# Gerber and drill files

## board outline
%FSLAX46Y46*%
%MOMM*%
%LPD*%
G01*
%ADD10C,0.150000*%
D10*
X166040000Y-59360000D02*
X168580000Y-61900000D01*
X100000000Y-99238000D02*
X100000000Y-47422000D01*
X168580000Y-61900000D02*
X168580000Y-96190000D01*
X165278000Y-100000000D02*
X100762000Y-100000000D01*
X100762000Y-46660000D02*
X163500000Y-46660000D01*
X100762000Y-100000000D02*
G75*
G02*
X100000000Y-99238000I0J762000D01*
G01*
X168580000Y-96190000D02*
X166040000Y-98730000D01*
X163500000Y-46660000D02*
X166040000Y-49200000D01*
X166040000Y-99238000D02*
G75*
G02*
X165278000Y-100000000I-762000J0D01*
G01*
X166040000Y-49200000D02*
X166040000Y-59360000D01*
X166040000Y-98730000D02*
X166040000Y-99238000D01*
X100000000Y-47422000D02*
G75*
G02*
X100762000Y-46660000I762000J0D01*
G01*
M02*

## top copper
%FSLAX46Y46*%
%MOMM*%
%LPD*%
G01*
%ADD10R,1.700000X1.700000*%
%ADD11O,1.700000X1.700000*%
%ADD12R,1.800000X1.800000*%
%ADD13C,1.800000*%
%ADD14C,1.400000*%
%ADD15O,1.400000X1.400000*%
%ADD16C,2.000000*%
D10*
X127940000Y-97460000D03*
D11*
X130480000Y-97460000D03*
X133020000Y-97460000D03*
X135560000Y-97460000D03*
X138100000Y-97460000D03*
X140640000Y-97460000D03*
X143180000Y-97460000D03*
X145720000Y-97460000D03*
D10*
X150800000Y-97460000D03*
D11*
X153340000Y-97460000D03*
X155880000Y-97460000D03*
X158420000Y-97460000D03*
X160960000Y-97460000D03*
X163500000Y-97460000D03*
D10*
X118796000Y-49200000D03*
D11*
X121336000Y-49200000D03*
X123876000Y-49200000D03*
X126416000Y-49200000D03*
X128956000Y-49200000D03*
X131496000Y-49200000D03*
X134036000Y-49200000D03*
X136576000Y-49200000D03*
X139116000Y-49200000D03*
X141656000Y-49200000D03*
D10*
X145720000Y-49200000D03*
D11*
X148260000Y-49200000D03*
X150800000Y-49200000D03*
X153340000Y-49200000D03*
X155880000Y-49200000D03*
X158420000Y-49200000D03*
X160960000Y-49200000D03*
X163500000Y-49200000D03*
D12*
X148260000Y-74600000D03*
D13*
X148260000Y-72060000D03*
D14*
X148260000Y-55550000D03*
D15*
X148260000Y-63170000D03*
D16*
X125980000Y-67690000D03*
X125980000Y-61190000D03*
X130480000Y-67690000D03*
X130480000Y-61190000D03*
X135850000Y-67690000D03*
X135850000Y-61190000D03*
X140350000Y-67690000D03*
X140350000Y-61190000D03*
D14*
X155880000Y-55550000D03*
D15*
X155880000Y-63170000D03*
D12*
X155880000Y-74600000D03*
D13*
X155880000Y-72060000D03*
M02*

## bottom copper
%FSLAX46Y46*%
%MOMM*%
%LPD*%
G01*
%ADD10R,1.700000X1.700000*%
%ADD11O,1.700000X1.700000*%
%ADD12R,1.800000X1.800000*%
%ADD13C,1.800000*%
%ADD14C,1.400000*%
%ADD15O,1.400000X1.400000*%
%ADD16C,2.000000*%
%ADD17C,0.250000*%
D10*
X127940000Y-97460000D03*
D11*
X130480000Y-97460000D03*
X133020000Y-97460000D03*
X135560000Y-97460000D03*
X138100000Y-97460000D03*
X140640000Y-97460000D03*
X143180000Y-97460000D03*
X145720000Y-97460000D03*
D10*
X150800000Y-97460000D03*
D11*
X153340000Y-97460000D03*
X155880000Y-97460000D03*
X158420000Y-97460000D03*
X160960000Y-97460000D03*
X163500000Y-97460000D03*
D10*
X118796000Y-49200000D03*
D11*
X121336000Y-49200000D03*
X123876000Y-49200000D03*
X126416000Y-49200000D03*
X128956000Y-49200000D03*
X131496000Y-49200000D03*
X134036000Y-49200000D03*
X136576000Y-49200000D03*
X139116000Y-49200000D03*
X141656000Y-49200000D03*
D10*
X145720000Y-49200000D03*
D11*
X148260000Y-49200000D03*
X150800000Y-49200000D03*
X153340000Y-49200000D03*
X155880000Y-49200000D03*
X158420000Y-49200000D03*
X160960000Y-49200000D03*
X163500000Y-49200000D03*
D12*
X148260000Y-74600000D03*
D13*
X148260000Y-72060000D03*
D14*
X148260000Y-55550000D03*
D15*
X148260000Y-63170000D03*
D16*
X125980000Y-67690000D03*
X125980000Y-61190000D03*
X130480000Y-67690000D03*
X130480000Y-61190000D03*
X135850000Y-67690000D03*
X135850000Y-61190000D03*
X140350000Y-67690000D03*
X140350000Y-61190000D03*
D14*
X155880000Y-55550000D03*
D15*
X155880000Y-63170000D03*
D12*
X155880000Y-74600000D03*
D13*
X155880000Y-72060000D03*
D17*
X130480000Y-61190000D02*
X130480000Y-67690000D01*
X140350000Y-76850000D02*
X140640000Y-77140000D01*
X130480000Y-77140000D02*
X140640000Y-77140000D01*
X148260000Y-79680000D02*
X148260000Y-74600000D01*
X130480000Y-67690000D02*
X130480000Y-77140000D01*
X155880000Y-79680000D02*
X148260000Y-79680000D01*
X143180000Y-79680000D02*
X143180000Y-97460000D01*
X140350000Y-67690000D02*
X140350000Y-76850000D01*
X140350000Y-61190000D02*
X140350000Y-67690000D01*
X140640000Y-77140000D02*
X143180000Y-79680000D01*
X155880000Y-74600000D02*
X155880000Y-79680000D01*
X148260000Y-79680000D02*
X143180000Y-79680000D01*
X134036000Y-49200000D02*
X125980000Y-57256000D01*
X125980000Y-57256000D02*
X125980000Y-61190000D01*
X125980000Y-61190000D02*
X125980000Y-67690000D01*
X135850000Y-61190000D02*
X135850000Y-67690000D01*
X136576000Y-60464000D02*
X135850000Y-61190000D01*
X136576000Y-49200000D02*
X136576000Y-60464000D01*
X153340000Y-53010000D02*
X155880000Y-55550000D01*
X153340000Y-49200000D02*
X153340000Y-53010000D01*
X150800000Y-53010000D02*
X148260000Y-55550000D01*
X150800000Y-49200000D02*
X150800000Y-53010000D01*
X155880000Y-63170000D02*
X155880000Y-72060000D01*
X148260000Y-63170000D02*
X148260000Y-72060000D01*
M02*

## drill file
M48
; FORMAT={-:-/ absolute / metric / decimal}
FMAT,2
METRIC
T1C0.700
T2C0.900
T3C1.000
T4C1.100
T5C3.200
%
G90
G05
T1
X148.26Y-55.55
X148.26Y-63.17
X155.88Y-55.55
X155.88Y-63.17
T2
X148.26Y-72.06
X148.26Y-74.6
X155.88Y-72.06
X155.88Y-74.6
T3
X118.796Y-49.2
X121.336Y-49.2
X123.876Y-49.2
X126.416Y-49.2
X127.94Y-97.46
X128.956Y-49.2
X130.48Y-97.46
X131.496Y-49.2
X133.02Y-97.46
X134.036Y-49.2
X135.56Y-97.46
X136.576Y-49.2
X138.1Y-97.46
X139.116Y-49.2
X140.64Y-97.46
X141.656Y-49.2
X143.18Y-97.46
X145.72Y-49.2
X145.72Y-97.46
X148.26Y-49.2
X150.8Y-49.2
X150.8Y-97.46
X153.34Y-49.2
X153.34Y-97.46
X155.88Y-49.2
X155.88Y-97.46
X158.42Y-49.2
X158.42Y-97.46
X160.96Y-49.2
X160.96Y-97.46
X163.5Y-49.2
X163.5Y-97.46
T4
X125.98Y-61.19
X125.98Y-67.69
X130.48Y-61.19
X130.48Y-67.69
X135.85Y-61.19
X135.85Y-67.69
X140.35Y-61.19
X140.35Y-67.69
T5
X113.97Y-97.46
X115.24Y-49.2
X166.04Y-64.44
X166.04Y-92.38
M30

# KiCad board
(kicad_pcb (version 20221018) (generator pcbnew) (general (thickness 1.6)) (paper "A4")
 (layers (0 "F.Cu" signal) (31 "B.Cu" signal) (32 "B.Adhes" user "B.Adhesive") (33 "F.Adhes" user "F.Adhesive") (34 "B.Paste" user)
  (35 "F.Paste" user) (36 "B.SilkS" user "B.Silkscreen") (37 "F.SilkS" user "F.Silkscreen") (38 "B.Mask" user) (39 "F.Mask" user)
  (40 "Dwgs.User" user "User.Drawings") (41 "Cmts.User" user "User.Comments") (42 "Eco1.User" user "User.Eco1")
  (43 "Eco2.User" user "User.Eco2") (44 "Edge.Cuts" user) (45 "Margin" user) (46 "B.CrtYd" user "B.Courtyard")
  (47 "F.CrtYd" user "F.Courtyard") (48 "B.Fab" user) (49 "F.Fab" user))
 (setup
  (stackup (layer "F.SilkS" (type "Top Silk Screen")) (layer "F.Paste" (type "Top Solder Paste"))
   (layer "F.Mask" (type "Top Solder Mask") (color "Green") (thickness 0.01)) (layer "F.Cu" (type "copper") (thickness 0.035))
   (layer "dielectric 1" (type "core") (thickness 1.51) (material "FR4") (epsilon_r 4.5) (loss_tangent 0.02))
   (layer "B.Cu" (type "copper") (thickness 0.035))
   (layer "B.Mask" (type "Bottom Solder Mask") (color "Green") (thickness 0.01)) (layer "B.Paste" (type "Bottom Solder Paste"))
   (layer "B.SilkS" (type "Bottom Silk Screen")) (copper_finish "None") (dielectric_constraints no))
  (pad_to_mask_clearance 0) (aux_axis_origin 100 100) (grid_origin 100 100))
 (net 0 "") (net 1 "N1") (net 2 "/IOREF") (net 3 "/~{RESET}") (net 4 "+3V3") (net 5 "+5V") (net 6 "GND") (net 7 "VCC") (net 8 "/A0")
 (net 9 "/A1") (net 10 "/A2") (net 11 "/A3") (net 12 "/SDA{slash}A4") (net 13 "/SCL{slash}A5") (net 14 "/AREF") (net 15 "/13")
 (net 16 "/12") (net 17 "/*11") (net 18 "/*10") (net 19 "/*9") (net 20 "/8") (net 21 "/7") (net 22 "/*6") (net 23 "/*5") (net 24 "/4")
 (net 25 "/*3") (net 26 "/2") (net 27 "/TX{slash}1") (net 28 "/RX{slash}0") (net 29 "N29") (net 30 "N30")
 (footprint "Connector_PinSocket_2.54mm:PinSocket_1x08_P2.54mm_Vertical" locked (layer "F.Cu") (at 127.94 97.46 90)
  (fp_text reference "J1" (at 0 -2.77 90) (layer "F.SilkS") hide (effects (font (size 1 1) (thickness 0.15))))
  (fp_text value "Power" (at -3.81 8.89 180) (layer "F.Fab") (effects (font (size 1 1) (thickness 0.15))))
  (pad "1" thru_hole rect locked (at 0 0 90) (size 1.7 1.7) (drill 1) (layers "*.Cu" "*.Mask") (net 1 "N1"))
  (pad "2" thru_hole oval locked (at 0 2.54 90) (size 1.7 1.7) (drill 1) (layers "*.Cu" "*.Mask") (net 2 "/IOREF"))
  (pad "3" thru_hole oval locked (at 0 5.08 90) (size 1.7 1.7) (drill 1) (layers "*.Cu" "*.Mask") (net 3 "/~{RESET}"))
  (pad "4" thru_hole oval locked (at 0 7.62 90) (size 1.7 1.7) (drill 1) (layers "*.Cu" "*.Mask") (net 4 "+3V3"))
  (pad "5" thru_hole oval locked (at 0 10.16 90) (size 1.7 1.7) (drill 1) (layers "*.Cu" "*.Mask") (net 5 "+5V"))
  (pad "6" thru_hole oval locked (at 0 12.7 90) (size 1.7 1.7) (drill 1) (layers "*.Cu" "*.Mask") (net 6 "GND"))
  (pad "7" thru_hole oval locked (at 0 15.24 90) (size 1.7 1.7) (drill 1) (layers "*.Cu" "*.Mask") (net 6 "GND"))
  (pad "8" thru_hole oval locked (at 0 17.78 90) (size 1.7 1.7) (drill 1) (layers "*.Cu" "*.Mask") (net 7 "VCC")))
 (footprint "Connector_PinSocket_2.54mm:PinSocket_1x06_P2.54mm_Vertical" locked (layer "F.Cu") (at 150.8 97.46 90)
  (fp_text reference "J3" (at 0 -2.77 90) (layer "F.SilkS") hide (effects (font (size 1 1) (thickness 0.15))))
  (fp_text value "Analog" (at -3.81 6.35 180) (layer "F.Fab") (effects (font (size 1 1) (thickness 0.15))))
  (pad "1" thru_hole rect locked (at 0 0 90) (size 1.7 1.7) (drill 1) (layers "*.Cu" "*.Mask") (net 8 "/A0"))
  (pad "2" thru_hole oval locked (at 0 2.54 90) (size 1.7 1.7) (drill 1) (layers "*.Cu" "*.Mask") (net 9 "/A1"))
  (pad "3" thru_hole oval locked (at 0 5.08 90) (size 1.7 1.7) (drill 1) (layers "*.Cu" "*.Mask") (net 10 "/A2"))
  (pad "4" thru_hole oval locked (at 0 7.62 90) (size 1.7 1.7) (drill 1) (layers "*.Cu" "*.Mask") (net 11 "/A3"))
  (pad "5" thru_hole oval locked (at 0 10.16 90) (size 1.7 1.7) (drill 1) (layers "*.Cu" "*.Mask") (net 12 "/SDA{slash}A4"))
  (pad "6" thru_hole oval locked (at 0 12.7 90) (size 1.7 1.7) (drill 1) (layers "*.Cu" "*.Mask") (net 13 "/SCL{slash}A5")))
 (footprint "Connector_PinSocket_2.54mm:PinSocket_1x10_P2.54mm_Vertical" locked (layer "F.Cu") (at 118.796 49.2 90)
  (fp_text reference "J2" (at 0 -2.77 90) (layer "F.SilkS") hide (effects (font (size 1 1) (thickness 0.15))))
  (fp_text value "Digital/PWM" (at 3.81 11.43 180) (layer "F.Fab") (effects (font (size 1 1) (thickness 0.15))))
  (pad "1" thru_hole rect locked (at 0 0 90) (size 1.7 1.7) (drill 1) (layers "*.Cu" "*.Mask") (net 13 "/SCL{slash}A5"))
  (pad "2" thru_hole oval locked (at 0 2.54 90) (size 1.7 1.7) (drill 1) (layers "*.Cu" "*.Mask") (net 12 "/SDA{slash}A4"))
  (pad "3" thru_hole oval locked (at 0 5.08 90) (size 1.7 1.7) (drill 1) (layers "*.Cu" "*.Mask") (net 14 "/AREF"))
  (pad "4" thru_hole oval locked (at 0 7.62 90) (size 1.7 1.7) (drill 1) (layers "*.Cu" "*.Mask") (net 6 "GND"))
  (pad "5" thru_hole oval locked (at 0 10.16 90) (size 1.7 1.7) (drill 1) (layers "*.Cu" "*.Mask") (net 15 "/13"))
  (pad "6" thru_hole oval locked (at 0 12.7 90) (size 1.7 1.7) (drill 1) (layers "*.Cu" "*.Mask") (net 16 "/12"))
  (pad "7" thru_hole oval locked (at 0 15.24 90) (size 1.7 1.7) (drill 1) (layers "*.Cu" "*.Mask") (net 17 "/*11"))
  (pad "8" thru_hole oval locked (at 0 17.78 90) (size 1.7 1.7) (drill 1) (layers "*.Cu" "*.Mask") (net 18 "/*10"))
  (pad "9" thru_hole oval locked (at 0 20.32 90) (size 1.7 1.7) (drill 1) (layers "*.Cu" "*.Mask") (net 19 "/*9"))
  (pad "10" thru_hole oval locked (at 0 22.86 90) (size 1.7 1.7) (drill 1) (layers "*.Cu" "*.Mask") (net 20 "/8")))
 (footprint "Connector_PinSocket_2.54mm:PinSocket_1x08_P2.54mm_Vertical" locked (layer "F.Cu") (at 145.72 49.2 90)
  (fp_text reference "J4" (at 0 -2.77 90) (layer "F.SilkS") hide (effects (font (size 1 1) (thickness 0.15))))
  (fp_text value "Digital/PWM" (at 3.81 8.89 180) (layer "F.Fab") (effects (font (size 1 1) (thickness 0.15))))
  (pad "1" thru_hole rect locked (at 0 0 90) (size 1.7 1.7) (drill 1) (layers "*.Cu" "*.Mask") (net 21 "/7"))
  (pad "2" thru_hole oval locked (at 0 2.54 90) (size 1.7 1.7) (drill 1) (layers "*.Cu" "*.Mask") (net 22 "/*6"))
  (pad "3" thru_hole oval locked (at 0 5.08 90) (size 1.7 1.7) (drill 1) (layers "*.Cu" "*.Mask") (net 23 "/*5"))
  (pad "4" thru_hole oval locked (at 0 7.62 90) (size 1.7 1.7) (drill 1) (layers "*.Cu" "*.Mask") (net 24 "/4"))
  (pad "5" thru_hole oval locked (at 0 10.16 90) (size 1.7 1.7) (drill 1) (layers "*.Cu" "*.Mask") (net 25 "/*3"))
  (pad "6" thru_hole oval locked (at 0 12.7 90) (size 1.7 1.7) (drill 1) (layers "*.Cu" "*.Mask") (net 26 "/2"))
  (pad "7" thru_hole oval locked (at 0 15.24 90) (size 1.7 1.7) (drill 1) (layers "*.Cu" "*.Mask") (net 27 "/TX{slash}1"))
  (pad "8" thru_hole oval locked (at 0 17.78 90) (size 1.7 1.7) (drill 1) (layers "*.Cu" "*.Mask") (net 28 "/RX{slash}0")))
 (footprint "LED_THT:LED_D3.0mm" (layer "F.Cu") (at 148.26 74.6 90)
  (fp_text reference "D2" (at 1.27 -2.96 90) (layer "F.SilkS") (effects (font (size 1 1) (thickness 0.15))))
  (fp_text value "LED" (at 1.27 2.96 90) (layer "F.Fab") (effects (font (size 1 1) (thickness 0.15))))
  (pad "1" thru_hole rect (at 0 0 90) (size 1.8 1.8) (drill 0.9) (layers "*.Cu" "*.Mask") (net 6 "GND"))
  (pad "2" thru_hole circle (at 2.54 0 90) (size 1.8 1.8) (drill 0.9) (layers "*.Cu" "*.Mask") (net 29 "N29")))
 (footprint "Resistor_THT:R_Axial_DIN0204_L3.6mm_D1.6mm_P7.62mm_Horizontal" (layer "F.Cu") (at 148.26 55.55 -90)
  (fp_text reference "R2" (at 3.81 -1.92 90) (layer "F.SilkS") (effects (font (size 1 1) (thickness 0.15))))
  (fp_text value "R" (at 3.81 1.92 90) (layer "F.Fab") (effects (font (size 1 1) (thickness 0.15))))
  (pad "1" thru_hole circle (at 0 0 270) (size 1.4 1.4) (drill 0.7) (layers "*.Cu" "*.Mask") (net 23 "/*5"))
  (pad "2" thru_hole oval (at 7.62 0 270) (size 1.4 1.4) (drill 0.7) (layers "*.Cu" "*.Mask") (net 29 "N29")))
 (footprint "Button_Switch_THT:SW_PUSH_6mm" (layer "F.Cu") (at 125.98 67.69 90)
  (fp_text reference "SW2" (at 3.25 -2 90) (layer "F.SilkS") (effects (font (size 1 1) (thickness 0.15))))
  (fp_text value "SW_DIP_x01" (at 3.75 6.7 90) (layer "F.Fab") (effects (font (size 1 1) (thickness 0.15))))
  (pad "1" thru_hole circle (at 0 0 180) (size 2 2) (drill 1.1) (layers "*.Cu" "*.Mask") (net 17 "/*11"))
  (pad "1" thru_hole circle (at 6.5 0 180) (size 2 2) (drill 1.1) (layers "*.Cu" "*.Mask") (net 17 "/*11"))
  (pad "2" thru_hole circle (at 0 4.5 180) (size 2 2) (drill 1.1) (layers "*.Cu" "*.Mask") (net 6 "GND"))
  (pad "2" thru_hole circle (at 6.5 4.5 180) (size 2 2) (drill 1.1) (layers "*.Cu" "*.Mask") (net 6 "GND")))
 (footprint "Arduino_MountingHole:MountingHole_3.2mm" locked (layer "F.Cu") (at 115.24 49.2)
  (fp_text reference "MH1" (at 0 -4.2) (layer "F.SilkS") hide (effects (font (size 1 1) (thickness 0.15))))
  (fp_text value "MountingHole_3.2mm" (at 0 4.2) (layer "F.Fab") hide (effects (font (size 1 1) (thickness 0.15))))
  (pad "" np_thru_hole circle locked (at 0 0) (size 3.2 3.2) (drill 3.2) (layers "*.Cu" "*.Mask")))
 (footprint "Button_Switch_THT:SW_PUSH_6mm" (layer "F.Cu") (at 135.85 67.69 90)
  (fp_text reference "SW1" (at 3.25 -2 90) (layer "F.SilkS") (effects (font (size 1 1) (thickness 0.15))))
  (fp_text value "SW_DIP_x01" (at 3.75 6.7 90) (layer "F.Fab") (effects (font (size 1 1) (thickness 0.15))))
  (pad "1" thru_hole circle (at 0 0 180) (size 2 2) (drill 1.1) (layers "*.Cu" "*.Mask") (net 18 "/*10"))
  (pad "1" thru_hole circle (at 6.5 0 180) (size 2 2) (drill 1.1) (layers "*.Cu" "*.Mask") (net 18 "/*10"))
  (pad "2" thru_hole circle (at 0 4.5 180) (size 2 2) (drill 1.1) (layers "*.Cu" "*.Mask") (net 6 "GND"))
  (pad "2" thru_hole circle (at 6.5 4.5 180) (size 2 2) (drill 1.1) (layers "*.Cu" "*.Mask") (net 6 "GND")))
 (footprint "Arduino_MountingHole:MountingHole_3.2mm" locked (layer "F.Cu") (at 113.97 97.46)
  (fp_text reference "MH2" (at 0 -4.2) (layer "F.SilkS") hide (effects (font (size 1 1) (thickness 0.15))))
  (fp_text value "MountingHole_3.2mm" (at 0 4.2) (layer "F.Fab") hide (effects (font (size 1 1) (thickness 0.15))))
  (pad "" np_thru_hole circle locked (at 0 0) (size 3.2 3.2) (drill 3.2) (layers "*.Cu" "*.Mask")))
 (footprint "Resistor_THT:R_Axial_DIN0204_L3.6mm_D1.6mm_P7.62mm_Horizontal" (layer "F.Cu") (at 155.88 55.55 -90)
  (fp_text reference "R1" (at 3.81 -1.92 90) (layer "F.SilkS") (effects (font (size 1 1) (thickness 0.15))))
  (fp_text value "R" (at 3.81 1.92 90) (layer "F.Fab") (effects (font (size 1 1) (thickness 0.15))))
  (pad "1" thru_hole circle (at 0 0 270) (size 1.4 1.4) (drill 0.7) (layers "*.Cu" "*.Mask") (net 24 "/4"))
  (pad "2" thru_hole oval (at 7.62 0 270) (size 1.4 1.4) (drill 0.7) (layers "*.Cu" "*.Mask") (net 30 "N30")))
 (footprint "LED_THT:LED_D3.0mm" (layer "F.Cu") (at 155.88 74.6 90)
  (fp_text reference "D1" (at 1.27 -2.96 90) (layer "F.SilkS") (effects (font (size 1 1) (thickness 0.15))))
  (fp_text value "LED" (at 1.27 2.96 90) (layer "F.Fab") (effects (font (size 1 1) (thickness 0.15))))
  (pad "1" thru_hole rect (at 0 0 90) (size 1.8 1.8) (drill 0.9) (layers "*.Cu" "*.Mask") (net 6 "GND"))
  (pad "2" thru_hole circle (at 2.54 0 90) (size 1.8 1.8) (drill 0.9) (layers "*.Cu" "*.Mask") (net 30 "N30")))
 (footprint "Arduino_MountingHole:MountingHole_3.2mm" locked (layer "F.Cu") (at 166.04 64.44)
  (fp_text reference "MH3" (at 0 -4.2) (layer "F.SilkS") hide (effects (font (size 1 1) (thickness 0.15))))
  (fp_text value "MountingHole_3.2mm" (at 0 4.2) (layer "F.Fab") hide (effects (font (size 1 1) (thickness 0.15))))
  (pad "" np_thru_hole circle locked (at 0 0) (size 3.2 3.2) (drill 3.2) (layers "*.Cu" "*.Mask")))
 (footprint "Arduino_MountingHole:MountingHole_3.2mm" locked (layer "F.Cu") (at 166.04 92.38)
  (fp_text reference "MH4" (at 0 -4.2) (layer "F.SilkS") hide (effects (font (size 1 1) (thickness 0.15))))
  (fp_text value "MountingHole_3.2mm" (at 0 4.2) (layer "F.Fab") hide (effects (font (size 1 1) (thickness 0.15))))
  (pad "" np_thru_hole circle locked (at 0 0) (size 3.2 3.2) (drill 3.2) (layers "*.Cu" "*.Mask")))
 (gr_line (start 166.04 59.36) (end 168.58 61.9) (stroke (width 0.15) (type solid)) (layer "Edge.Cuts"))
 (gr_line (start 100 99.238) (end 100 47.422) (stroke (width 0.15) (type solid)) (layer "Edge.Cuts"))
 (gr_line (start 168.58 61.9) (end 168.58 96.19) (stroke (width 0.15) (type solid)) (layer "Edge.Cuts"))
 (gr_line (start 165.278 100) (end 100.762 100) (stroke (width 0.15) (type solid)) (layer "Edge.Cuts"))
 (gr_line (start 100.762 46.66) (end 163.5 46.66) (stroke (width 0.15) (type solid)) (layer "Edge.Cuts"))
 (gr_arc (start 100.762 100) (mid 100.223185 99.776815) (end 100 99.238) (stroke (width 0.15) (type solid)) (layer "Edge.Cuts"))
 (gr_line (start 168.58 96.19) (end 166.04 98.73) (stroke (width 0.15) (type solid)) (layer "Edge.Cuts"))
 (gr_line (start 163.5 46.66) (end 166.04 49.2) (stroke (width 0.15) (type solid)) (layer "Edge.Cuts"))
 (gr_arc (start 166.04 99.238) (mid 165.816815 99.776815) (end 165.278 100) (stroke (width 0.15) (type solid)) (layer "Edge.Cuts"))
 (gr_line (start 166.04 49.2) (end 166.04 59.36) (stroke (width 0.15) (type solid)) (layer "Edge.Cuts"))
 (gr_line (start 166.04 98.73) (end 166.04 99.238) (stroke (width 0.15) (type solid)) (layer "Edge.Cuts"))
 (gr_arc (start 100 47.422) (mid 100.223185 46.883185) (end 100.762 46.66) (stroke (width 0.15) (type solid)) (layer "Edge.Cuts"))
 (segment (start 130.48 61.19) (end 130.48 67.69) (width 0.25) (layer "B.Cu") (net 6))
 (segment (start 140.35 76.85) (end 140.64 77.14) (width 0.25) (layer "B.Cu") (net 6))
 (segment (start 130.48 77.14) (end 140.64 77.14) (width 0.25) (layer "B.Cu") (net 6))
 (segment (start 148.26 79.68) (end 148.26 74.6) (width 0.25) (layer "B.Cu") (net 6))
 (segment (start 130.48 67.69) (end 130.48 77.14) (width 0.25) (layer "B.Cu") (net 6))
 (segment (start 155.88 79.68) (end 148.26 79.68) (width 0.25) (layer "B.Cu") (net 6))
 (segment (start 143.18 79.68) (end 143.18 97.46) (width 0.25) (layer "B.Cu") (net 6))
 (segment (start 140.35 67.69) (end 140.35 76.85) (width 0.25) (layer "B.Cu") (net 6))
 (segment (start 140.35 61.19) (end 140.35 67.69) (width 0.25) (layer "B.Cu") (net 6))
 (segment (start 140.64 77.14) (end 143.18 79.68) (width 0.25) (layer "B.Cu") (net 6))
 (segment (start 155.88 74.6) (end 155.88 79.68) (width 0.25) (layer "B.Cu") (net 6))
 (segment (start 148.26 79.68) (end 143.18 79.68) (width 0.25) (layer "B.Cu") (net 6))
 (segment (start 134.036 49.2) (end 125.98 57.256) (width 0.25) (layer "B.Cu") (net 17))
 (segment (start 125.98 57.256) (end 125.98 61.19) (width 0.25) (layer "B.Cu") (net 17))
 (segment (start 125.98 61.19) (end 125.98 67.69) (width 0.25) (layer "B.Cu") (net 17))
 (segment (start 135.85 61.19) (end 135.85 67.69) (width 0.25) (layer "B.Cu") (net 18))
 (segment (start 136.576 60.464) (end 135.85 61.19) (width 0.25) (layer "B.Cu") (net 18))
 (segment (start 136.576 49.2) (end 136.576 60.464) (width 0.25) (layer "B.Cu") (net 18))
 (segment (start 153.34 53.01) (end 155.88 55.55) (width 0.25) (layer "B.Cu") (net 24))
 (segment (start 153.34 49.2) (end 153.34 53.01) (width 0.25) (layer "B.Cu") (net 24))
 (segment (start 150.8 53.01) (end 148.26 55.55) (width 0.25) (layer "B.Cu") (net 23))
 (segment (start 150.8 49.2) (end 150.8 53.01) (width 0.25) (layer "B.Cu") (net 23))
 (segment (start 155.88 63.17) (end 155.88 72.06) (width 0.25) (layer "B.Cu") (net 30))
 (segment (start 148.26 63.17) (end 148.26 72.06) (width 0.25) (layer "B.Cu") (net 29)))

